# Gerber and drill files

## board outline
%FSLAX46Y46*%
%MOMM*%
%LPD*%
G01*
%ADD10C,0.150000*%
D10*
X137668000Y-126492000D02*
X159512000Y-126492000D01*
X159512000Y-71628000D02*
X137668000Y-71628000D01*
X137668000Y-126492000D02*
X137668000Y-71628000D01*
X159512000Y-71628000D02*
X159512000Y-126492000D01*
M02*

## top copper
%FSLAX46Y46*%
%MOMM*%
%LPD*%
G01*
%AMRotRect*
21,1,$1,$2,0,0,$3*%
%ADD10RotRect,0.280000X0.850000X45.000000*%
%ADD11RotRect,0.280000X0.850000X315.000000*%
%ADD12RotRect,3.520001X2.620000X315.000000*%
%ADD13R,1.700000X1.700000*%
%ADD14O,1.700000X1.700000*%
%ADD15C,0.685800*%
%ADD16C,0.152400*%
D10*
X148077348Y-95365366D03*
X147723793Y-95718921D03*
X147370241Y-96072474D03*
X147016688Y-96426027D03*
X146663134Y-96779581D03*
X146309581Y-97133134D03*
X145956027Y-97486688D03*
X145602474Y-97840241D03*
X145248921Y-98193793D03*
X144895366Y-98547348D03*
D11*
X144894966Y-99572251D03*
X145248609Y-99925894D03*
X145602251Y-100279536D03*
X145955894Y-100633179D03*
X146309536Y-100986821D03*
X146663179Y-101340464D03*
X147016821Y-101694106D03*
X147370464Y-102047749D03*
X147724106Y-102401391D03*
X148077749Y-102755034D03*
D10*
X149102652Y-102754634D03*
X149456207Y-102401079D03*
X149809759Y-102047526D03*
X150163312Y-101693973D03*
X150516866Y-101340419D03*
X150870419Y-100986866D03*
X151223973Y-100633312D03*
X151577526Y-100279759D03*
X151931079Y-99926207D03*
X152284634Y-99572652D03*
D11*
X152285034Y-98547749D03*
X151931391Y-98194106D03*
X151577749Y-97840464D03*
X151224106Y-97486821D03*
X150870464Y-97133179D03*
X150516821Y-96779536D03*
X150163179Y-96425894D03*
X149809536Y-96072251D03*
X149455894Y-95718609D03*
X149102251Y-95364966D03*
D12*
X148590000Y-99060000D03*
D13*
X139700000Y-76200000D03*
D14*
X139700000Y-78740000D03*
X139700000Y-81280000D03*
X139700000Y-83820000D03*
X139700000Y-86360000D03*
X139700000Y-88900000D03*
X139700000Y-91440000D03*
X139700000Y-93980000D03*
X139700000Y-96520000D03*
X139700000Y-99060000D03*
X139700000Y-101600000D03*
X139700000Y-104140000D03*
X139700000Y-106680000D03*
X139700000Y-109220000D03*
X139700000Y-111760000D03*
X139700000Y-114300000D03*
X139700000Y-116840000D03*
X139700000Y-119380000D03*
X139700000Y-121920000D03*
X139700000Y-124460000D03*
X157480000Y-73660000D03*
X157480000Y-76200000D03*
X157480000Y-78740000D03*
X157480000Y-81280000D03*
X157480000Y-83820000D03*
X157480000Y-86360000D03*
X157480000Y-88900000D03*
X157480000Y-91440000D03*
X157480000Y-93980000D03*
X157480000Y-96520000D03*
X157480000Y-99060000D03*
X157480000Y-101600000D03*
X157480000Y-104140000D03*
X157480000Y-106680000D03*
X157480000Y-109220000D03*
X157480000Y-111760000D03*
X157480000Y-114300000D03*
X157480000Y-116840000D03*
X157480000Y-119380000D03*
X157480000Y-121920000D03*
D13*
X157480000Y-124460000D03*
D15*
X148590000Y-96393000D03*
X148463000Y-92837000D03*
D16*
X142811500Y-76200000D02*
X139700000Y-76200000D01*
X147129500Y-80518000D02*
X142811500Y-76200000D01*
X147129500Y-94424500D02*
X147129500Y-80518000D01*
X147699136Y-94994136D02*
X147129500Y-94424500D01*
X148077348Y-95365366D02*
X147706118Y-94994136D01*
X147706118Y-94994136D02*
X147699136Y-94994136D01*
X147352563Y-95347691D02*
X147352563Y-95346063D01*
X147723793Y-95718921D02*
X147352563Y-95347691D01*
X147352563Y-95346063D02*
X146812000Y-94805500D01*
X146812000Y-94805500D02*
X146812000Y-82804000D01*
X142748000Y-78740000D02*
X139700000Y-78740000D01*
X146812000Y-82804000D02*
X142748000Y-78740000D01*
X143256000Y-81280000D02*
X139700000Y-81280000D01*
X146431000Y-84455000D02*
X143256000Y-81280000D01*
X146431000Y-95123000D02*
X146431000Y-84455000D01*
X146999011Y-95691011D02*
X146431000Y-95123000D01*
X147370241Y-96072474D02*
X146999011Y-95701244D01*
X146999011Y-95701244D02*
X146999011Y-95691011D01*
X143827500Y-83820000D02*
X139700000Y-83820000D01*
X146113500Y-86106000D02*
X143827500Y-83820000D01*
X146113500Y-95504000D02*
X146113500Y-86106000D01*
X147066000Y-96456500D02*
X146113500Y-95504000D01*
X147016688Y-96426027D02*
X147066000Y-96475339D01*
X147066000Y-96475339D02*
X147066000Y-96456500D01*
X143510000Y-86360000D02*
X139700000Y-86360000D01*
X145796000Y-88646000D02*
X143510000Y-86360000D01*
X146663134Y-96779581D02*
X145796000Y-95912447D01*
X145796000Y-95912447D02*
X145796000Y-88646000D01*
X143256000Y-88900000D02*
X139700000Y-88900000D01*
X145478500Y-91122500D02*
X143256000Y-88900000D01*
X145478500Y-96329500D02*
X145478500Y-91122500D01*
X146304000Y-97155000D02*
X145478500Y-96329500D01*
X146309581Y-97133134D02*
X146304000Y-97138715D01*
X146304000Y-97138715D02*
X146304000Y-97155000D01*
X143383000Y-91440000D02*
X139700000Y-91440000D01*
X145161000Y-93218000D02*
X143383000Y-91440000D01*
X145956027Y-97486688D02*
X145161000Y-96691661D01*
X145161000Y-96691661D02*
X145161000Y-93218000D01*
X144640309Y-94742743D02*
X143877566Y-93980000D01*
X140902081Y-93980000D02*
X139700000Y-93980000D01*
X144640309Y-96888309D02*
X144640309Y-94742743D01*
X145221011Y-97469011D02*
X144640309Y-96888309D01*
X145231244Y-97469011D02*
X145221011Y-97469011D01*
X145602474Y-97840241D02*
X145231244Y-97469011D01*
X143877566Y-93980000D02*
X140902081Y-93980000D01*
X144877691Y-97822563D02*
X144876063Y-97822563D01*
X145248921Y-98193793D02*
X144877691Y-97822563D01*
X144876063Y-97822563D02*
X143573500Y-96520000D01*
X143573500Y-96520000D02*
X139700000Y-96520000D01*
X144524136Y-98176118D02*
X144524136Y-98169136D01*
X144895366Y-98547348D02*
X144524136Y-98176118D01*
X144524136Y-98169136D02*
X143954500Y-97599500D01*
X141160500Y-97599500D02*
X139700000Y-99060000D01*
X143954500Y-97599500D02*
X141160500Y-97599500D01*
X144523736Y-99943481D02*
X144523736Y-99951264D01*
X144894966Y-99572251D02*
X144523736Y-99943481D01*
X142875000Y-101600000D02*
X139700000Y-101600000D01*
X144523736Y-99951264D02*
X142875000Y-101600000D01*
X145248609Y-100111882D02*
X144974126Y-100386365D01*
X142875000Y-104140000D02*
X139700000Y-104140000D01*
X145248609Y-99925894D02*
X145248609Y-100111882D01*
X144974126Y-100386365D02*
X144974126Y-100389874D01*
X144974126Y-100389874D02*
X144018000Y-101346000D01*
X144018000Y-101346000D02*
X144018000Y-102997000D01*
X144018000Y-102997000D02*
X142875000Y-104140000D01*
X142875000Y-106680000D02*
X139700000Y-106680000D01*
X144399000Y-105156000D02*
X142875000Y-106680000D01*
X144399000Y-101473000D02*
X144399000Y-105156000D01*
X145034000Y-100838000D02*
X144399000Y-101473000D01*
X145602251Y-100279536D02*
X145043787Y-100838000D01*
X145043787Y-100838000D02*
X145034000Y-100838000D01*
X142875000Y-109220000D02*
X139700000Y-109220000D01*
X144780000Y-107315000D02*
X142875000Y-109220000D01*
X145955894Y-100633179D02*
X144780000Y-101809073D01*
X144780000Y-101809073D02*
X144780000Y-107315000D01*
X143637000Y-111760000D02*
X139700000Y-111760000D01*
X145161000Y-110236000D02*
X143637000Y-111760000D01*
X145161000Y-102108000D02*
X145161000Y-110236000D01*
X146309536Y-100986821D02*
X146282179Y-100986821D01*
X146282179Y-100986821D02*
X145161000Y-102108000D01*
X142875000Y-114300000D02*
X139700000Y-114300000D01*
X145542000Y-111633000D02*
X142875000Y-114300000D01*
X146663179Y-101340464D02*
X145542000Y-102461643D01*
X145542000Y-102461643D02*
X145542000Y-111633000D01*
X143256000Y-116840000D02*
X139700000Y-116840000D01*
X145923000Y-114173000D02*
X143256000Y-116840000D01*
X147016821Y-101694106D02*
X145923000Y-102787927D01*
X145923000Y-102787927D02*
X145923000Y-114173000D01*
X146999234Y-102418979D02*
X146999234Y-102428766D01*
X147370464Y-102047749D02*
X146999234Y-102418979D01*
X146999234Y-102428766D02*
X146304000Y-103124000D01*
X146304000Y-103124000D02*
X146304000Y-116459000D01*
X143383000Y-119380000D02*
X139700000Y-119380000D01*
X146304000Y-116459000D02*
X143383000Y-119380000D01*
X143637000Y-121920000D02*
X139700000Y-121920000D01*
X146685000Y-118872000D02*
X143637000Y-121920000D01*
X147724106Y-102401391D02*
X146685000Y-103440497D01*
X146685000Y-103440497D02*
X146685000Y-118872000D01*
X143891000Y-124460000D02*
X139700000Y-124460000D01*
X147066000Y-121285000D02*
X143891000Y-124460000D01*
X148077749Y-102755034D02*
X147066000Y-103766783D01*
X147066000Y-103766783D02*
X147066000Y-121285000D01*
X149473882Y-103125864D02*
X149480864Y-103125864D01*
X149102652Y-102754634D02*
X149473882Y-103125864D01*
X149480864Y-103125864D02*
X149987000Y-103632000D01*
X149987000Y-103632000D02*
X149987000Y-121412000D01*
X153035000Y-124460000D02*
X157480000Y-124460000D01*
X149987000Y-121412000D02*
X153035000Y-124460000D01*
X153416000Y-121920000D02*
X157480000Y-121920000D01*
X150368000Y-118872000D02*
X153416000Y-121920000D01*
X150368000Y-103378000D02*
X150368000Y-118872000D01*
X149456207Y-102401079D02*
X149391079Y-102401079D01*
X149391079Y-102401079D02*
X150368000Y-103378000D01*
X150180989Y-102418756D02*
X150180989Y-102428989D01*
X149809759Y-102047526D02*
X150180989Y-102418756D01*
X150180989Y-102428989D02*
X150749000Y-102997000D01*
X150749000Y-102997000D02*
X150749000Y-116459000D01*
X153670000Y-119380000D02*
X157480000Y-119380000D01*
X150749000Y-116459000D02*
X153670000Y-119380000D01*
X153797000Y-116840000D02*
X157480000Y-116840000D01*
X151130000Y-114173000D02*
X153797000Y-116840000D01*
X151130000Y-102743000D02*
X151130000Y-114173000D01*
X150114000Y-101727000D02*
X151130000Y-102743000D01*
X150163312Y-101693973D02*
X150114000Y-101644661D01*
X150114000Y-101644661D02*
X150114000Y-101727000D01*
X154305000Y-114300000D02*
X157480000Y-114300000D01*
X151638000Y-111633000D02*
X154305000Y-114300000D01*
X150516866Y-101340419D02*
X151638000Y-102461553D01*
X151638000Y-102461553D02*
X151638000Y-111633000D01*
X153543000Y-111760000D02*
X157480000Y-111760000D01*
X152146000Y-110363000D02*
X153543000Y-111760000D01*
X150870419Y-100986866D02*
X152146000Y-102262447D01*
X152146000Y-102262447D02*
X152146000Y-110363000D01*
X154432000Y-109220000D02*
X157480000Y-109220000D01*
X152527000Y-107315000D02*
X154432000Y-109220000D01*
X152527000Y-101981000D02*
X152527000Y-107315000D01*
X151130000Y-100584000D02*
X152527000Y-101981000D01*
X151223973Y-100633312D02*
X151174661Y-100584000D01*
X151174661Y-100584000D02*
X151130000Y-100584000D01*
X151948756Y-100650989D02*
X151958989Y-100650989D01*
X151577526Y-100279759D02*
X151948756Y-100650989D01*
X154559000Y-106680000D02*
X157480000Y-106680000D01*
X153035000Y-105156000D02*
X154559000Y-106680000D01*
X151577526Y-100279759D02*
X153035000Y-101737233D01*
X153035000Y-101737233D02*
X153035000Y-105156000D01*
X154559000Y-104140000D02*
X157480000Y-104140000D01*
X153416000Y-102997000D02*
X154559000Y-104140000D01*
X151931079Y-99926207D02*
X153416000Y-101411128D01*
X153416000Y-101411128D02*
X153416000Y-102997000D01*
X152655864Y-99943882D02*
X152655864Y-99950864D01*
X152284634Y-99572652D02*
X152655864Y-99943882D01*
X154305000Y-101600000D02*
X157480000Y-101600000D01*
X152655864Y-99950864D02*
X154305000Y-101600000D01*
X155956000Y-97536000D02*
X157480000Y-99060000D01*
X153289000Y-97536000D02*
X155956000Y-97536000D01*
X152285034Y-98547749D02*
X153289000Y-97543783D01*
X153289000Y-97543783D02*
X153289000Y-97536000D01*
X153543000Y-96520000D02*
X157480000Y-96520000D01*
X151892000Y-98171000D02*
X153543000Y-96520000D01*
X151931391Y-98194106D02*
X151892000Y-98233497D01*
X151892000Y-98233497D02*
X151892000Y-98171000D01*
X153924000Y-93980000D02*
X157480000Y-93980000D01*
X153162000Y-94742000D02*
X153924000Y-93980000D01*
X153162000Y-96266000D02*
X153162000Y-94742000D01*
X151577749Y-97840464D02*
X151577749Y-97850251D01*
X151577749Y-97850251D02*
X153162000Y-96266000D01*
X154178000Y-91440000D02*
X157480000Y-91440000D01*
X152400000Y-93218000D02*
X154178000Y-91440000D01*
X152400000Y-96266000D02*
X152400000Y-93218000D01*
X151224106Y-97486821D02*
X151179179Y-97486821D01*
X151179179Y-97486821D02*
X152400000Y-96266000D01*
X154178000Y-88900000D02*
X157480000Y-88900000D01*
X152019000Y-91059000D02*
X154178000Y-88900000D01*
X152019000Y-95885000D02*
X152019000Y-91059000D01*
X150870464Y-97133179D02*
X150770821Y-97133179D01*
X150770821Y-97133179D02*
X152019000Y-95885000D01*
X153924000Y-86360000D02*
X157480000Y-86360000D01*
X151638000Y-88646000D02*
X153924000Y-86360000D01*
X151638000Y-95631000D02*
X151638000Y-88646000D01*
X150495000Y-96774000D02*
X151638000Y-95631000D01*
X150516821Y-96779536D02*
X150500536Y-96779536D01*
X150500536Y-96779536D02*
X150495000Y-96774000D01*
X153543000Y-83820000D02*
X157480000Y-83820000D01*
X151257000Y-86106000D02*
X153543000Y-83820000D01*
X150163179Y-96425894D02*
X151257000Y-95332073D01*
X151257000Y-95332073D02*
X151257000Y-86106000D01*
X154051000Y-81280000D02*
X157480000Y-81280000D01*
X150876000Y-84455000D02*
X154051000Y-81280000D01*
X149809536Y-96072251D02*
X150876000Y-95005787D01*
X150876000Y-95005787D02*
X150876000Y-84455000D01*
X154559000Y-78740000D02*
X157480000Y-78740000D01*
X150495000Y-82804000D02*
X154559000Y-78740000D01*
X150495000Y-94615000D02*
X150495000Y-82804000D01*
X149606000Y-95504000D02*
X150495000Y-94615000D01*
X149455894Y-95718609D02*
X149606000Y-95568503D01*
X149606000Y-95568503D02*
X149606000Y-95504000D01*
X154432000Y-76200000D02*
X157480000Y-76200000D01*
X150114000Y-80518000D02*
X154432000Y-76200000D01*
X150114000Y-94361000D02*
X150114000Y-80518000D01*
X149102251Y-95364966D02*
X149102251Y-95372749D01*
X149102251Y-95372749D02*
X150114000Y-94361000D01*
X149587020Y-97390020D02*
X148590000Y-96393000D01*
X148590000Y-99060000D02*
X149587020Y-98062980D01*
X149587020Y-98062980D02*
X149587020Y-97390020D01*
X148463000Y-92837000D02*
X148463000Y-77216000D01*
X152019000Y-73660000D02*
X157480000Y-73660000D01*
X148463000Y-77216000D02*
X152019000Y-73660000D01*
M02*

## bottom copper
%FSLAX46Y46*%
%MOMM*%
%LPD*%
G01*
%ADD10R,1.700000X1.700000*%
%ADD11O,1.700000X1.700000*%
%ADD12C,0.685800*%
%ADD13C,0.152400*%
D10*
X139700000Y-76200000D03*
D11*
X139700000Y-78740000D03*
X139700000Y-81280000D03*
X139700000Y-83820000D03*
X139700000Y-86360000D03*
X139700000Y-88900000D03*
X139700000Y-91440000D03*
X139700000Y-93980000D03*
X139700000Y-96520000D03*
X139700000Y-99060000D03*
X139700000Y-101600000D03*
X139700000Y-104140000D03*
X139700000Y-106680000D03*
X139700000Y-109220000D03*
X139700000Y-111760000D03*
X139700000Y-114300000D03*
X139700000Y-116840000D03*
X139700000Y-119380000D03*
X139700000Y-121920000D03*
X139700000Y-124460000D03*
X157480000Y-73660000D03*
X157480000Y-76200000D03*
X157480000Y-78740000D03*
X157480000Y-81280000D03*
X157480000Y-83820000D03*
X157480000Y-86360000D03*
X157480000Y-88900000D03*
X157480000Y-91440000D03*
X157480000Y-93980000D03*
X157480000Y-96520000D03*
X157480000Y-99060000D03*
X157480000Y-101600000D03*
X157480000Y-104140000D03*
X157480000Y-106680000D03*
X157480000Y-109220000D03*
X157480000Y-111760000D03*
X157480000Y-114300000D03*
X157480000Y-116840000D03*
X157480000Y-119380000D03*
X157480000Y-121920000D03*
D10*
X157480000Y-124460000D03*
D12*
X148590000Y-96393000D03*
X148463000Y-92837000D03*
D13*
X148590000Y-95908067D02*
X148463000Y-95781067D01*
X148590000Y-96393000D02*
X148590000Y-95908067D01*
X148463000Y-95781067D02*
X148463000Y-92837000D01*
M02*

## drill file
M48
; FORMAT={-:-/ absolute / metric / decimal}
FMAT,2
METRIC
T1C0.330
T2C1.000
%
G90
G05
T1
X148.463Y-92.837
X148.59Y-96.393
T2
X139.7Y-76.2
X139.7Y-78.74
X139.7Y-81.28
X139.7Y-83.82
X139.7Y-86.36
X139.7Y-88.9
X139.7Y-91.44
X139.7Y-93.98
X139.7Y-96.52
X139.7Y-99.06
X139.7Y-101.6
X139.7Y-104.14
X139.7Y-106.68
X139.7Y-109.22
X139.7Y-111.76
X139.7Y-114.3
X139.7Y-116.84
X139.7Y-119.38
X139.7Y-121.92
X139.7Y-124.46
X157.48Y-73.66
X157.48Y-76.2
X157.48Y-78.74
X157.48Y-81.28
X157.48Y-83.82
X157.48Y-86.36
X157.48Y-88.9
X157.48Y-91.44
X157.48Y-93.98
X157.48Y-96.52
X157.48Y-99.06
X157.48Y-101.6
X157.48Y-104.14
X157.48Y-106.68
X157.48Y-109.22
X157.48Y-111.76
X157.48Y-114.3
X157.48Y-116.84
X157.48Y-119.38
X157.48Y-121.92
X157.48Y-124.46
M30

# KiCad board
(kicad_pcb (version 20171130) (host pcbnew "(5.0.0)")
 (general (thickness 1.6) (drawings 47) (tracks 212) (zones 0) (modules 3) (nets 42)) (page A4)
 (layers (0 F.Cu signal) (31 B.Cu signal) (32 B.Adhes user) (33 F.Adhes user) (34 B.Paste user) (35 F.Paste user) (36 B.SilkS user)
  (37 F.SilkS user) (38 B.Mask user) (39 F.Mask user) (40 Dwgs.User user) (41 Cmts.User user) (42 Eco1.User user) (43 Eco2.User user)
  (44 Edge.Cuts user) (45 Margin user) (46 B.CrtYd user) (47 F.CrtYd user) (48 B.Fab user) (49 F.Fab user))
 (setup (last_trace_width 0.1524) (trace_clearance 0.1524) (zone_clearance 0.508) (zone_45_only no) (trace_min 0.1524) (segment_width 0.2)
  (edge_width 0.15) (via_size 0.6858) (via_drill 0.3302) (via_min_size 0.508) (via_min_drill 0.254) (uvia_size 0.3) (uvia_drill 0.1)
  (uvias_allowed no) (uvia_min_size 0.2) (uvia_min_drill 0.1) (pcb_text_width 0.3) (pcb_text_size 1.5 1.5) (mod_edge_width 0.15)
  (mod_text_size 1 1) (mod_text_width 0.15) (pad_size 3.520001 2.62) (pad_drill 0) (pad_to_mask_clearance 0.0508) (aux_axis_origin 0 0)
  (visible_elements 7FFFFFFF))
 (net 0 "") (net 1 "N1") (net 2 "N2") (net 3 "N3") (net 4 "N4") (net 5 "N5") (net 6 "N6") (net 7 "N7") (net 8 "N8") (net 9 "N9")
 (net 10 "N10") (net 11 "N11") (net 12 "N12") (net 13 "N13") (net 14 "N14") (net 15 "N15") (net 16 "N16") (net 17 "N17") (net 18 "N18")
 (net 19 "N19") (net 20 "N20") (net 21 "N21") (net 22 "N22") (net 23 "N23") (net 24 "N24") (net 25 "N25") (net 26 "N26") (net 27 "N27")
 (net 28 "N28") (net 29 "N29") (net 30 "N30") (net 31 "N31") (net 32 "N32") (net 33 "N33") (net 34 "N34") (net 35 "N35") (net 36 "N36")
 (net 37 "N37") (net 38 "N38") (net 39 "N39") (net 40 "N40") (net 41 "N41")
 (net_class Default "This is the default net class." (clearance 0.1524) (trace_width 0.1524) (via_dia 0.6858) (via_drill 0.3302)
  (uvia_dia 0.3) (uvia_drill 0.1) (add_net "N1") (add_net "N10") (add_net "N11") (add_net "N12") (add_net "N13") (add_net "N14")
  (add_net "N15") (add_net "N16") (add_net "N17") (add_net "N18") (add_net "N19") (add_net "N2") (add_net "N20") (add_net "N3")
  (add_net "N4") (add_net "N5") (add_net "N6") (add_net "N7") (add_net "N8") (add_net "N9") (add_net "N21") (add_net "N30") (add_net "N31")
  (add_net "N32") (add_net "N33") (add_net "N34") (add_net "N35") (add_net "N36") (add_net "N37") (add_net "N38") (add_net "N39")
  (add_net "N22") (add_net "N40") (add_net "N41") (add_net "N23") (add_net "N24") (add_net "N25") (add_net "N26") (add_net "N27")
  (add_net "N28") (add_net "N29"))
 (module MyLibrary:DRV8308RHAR (layer F.Cu) (at 148.59 99.06 315)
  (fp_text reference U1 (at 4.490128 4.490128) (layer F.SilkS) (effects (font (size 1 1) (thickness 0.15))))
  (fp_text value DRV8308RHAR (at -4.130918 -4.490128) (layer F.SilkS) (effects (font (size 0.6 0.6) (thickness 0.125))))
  (pad 1 smd rect (at -2.975 -2.250001 45) (size 0.28 0.85) (layers F.Cu F.Paste F.Mask) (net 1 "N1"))
  (pad 2 smd rect (at -2.975 -1.749999 45) (size 0.28 0.85) (layers F.Cu F.Paste F.Mask) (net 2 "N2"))
  (pad 3 smd rect (at -2.975 -1.25 45) (size 0.28 0.85) (layers F.Cu F.Paste F.Mask) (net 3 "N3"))
  (pad 4 smd rect (at -2.975 -0.750001 45) (size 0.28 0.85) (layers F.Cu F.Paste F.Mask) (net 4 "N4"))
  (pad 5 smd rect (at -2.975 -0.25 45) (size 0.28 0.85) (layers F.Cu F.Paste F.Mask) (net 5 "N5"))
  (pad 6 smd rect (at -2.975 0.25 45) (size 0.28 0.85) (layers F.Cu F.Paste F.Mask) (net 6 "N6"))
  (pad 7 smd rect (at -2.975 0.750001 45) (size 0.28 0.85) (layers F.Cu F.Paste F.Mask) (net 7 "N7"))
  (pad 8 smd rect (at -2.975 1.25 45) (size 0.28 0.85) (layers F.Cu F.Paste F.Mask) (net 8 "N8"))
  (pad 9 smd rect (at -2.975 1.749999 45) (size 0.28 0.85) (layers F.Cu F.Paste F.Mask) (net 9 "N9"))
  (pad 10 smd rect (at -2.975 2.250001 45) (size 0.28 0.85) (layers F.Cu F.Paste F.Mask) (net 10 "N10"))
  (pad 11 smd rect (at -2.250567 2.975 315) (size 0.28 0.85) (layers F.Cu F.Paste F.Mask) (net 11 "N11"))
  (pad 12 smd rect (at -1.750441 2.975 315) (size 0.28 0.85) (layers F.Cu F.Paste F.Mask) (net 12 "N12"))
  (pad 13 smd rect (at -1.250315 2.975 315) (size 0.28 0.85) (layers F.Cu F.Paste F.Mask) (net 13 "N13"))
  (pad 14 smd rect (at -0.750189 2.975 315) (size 0.28 0.85) (layers F.Cu F.Paste F.Mask) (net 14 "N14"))
  (pad 15 smd rect (at -0.250063 2.975 315) (size 0.28 0.85) (layers F.Cu F.Paste F.Mask) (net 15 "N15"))
  (pad 16 smd rect (at 0.250063 2.975 315) (size 0.28 0.85) (layers F.Cu F.Paste F.Mask) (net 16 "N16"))
  (pad 17 smd rect (at 0.750189 2.975 315) (size 0.28 0.85) (layers F.Cu F.Paste F.Mask) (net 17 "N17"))
  (pad 18 smd rect (at 1.250315 2.975 315) (size 0.28 0.85) (layers F.Cu F.Paste F.Mask) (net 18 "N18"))
  (pad 19 smd rect (at 1.750441 2.975 315) (size 0.28 0.85) (layers F.Cu F.Paste F.Mask) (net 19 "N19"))
  (pad 20 smd rect (at 2.250567 2.975 315) (size 0.28 0.85) (layers F.Cu F.Paste F.Mask) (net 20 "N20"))
  (pad 21 smd rect (at 2.975 2.250001 45) (size 0.28 0.85) (layers F.Cu F.Paste F.Mask) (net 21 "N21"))
  (pad 22 smd rect (at 2.975 1.749999 45) (size 0.28 0.85) (layers F.Cu F.Paste F.Mask) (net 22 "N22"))
  (pad 23 smd rect (at 2.975 1.25 45) (size 0.28 0.85) (layers F.Cu F.Paste F.Mask) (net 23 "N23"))
  (pad 24 smd rect (at 2.975 0.750001 45) (size 0.28 0.85) (layers F.Cu F.Paste F.Mask) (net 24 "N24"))
  (pad 25 smd rect (at 2.975 0.25 45) (size 0.28 0.85) (layers F.Cu F.Paste F.Mask) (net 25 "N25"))
  (pad 26 smd rect (at 2.975 -0.25 45) (size 0.28 0.85) (layers F.Cu F.Paste F.Mask) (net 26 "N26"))
  (pad 27 smd rect (at 2.975 -0.750001 45) (size 0.28 0.85) (layers F.Cu F.Paste F.Mask) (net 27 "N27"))
  (pad 28 smd rect (at 2.975 -1.25 45) (size 0.28 0.85) (layers F.Cu F.Paste F.Mask) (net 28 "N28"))
  (pad 29 smd rect (at 2.975 -1.749999 45) (size 0.28 0.85) (layers F.Cu F.Paste F.Mask) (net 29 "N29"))
  (pad 30 smd rect (at 2.975 -2.250001 45) (size 0.28 0.85) (layers F.Cu F.Paste F.Mask) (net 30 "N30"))
  (pad 31 smd rect (at 2.250567 -2.975 315) (size 0.28 0.85) (layers F.Cu F.Paste F.Mask) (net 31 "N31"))
  (pad 32 smd rect (at 1.750441 -2.975 315) (size 0.28 0.85) (layers F.Cu F.Paste F.Mask) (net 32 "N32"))
  (pad 33 smd rect (at 1.250315 -2.975 315) (size 0.28 0.85) (layers F.Cu F.Paste F.Mask) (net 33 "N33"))
  (pad 34 smd rect (at 0.750189 -2.975 315) (size 0.28 0.85) (layers F.Cu F.Paste F.Mask) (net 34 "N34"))
  (pad 35 smd rect (at 0.250063 -2.975 315) (size 0.28 0.85) (layers F.Cu F.Paste F.Mask) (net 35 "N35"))
  (pad 36 smd rect (at -0.250063 -2.975 315) (size 0.28 0.85) (layers F.Cu F.Paste F.Mask) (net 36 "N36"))
  (pad 37 smd rect (at -0.750189 -2.975 315) (size 0.28 0.85) (layers F.Cu F.Paste F.Mask) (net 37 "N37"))
  (pad 38 smd rect (at -1.250315 -2.975 315) (size 0.28 0.85) (layers F.Cu F.Paste F.Mask) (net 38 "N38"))
  (pad 39 smd rect (at -1.750441 -2.975 315) (size 0.28 0.85) (layers F.Cu F.Paste F.Mask) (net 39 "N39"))
  (pad 40 smd rect (at -2.250567 -2.975 315) (size 0.28 0.85) (layers F.Cu F.Paste F.Mask) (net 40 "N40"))
  (pad 41 smd rect (at 0 0 315) (size 3.520001 2.62) (layers F.Cu F.Paste F.Mask) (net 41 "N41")))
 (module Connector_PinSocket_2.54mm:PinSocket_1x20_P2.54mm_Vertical (layer F.Cu) (at 139.7 76.2)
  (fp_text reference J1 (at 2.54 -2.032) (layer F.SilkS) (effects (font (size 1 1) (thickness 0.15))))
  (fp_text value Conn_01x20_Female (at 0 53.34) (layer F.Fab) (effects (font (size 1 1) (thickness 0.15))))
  (pad 1 thru_hole rect (at 0 0) (size 1.7 1.7) (drill 1) (layers *.Cu *.Mask) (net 1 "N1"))
  (pad 2 thru_hole oval (at 0 2.54) (size 1.7 1.7) (drill 1) (layers *.Cu *.Mask) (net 2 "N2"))
  (pad 3 thru_hole oval (at 0 5.08) (size 1.7 1.7) (drill 1) (layers *.Cu *.Mask) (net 3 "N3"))
  (pad 4 thru_hole oval (at 0 7.62) (size 1.7 1.7) (drill 1) (layers *.Cu *.Mask) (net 4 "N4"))
  (pad 5 thru_hole oval (at 0 10.16) (size 1.7 1.7) (drill 1) (layers *.Cu *.Mask) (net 5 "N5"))
  (pad 6 thru_hole oval (at 0 12.7) (size 1.7 1.7) (drill 1) (layers *.Cu *.Mask) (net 6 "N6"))
  (pad 7 thru_hole oval (at 0 15.24) (size 1.7 1.7) (drill 1) (layers *.Cu *.Mask) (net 7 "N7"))
  (pad 8 thru_hole oval (at 0 17.78) (size 1.7 1.7) (drill 1) (layers *.Cu *.Mask) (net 8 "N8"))
  (pad 9 thru_hole oval (at 0 20.32) (size 1.7 1.7) (drill 1) (layers *.Cu *.Mask) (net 9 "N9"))
  (pad 10 thru_hole oval (at 0 22.86) (size 1.7 1.7) (drill 1) (layers *.Cu *.Mask) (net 10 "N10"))
  (pad 11 thru_hole oval (at 0 25.4) (size 1.7 1.7) (drill 1) (layers *.Cu *.Mask) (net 11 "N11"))
  (pad 12 thru_hole oval (at 0 27.94) (size 1.7 1.7) (drill 1) (layers *.Cu *.Mask) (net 12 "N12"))
  (pad 13 thru_hole oval (at 0 30.48) (size 1.7 1.7) (drill 1) (layers *.Cu *.Mask) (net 13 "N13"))
  (pad 14 thru_hole oval (at 0 33.02) (size 1.7 1.7) (drill 1) (layers *.Cu *.Mask) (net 14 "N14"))
  (pad 15 thru_hole oval (at 0 35.56) (size 1.7 1.7) (drill 1) (layers *.Cu *.Mask) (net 15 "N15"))
  (pad 16 thru_hole oval (at 0 38.1) (size 1.7 1.7) (drill 1) (layers *.Cu *.Mask) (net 16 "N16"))
  (pad 17 thru_hole oval (at 0 40.64) (size 1.7 1.7) (drill 1) (layers *.Cu *.Mask) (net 17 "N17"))
  (pad 18 thru_hole oval (at 0 43.18) (size 1.7 1.7) (drill 1) (layers *.Cu *.Mask) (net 18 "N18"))
  (pad 19 thru_hole oval (at 0 45.72) (size 1.7 1.7) (drill 1) (layers *.Cu *.Mask) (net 19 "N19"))
  (pad 20 thru_hole oval (at 0 48.26) (size 1.7 1.7) (drill 1) (layers *.Cu *.Mask) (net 20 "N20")))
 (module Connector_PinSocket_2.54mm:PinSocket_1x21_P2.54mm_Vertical (layer F.Cu) (at 157.48 124.46 180)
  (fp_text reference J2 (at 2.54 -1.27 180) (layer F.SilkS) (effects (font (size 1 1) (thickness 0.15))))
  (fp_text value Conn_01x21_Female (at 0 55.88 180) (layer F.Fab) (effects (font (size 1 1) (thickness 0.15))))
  (pad 21 thru_hole oval (at 0 50.8 180) (size 1.7 1.7) (drill 1) (layers *.Cu *.Mask) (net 41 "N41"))
  (pad 20 thru_hole oval (at 0 48.26 180) (size 1.7 1.7) (drill 1) (layers *.Cu *.Mask) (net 40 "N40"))
  (pad 19 thru_hole oval (at 0 45.72 180) (size 1.7 1.7) (drill 1) (layers *.Cu *.Mask) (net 39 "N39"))
  (pad 18 thru_hole oval (at 0 43.18 180) (size 1.7 1.7) (drill 1) (layers *.Cu *.Mask) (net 38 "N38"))
  (pad 17 thru_hole oval (at 0 40.64 180) (size 1.7 1.7) (drill 1) (layers *.Cu *.Mask) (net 37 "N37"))
  (pad 16 thru_hole oval (at 0 38.1 180) (size 1.7 1.7) (drill 1) (layers *.Cu *.Mask) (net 36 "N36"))
  (pad 15 thru_hole oval (at 0 35.56 180) (size 1.7 1.7) (drill 1) (layers *.Cu *.Mask) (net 35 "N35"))
  (pad 14 thru_hole oval (at 0 33.02 180) (size 1.7 1.7) (drill 1) (layers *.Cu *.Mask) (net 34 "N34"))
  (pad 13 thru_hole oval (at 0 30.48 180) (size 1.7 1.7) (drill 1) (layers *.Cu *.Mask) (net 33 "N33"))
  (pad 12 thru_hole oval (at 0 27.94 180) (size 1.7 1.7) (drill 1) (layers *.Cu *.Mask) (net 32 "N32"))
  (pad 11 thru_hole oval (at 0 25.4 180) (size 1.7 1.7) (drill 1) (layers *.Cu *.Mask) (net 31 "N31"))
  (pad 10 thru_hole oval (at 0 22.86 180) (size 1.7 1.7) (drill 1) (layers *.Cu *.Mask) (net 30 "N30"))
  (pad 9 thru_hole oval (at 0 20.32 180) (size 1.7 1.7) (drill 1) (layers *.Cu *.Mask) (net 29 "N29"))
  (pad 8 thru_hole oval (at 0 17.78 180) (size 1.7 1.7) (drill 1) (layers *.Cu *.Mask) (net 28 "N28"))
  (pad 7 thru_hole oval (at 0 15.24 180) (size 1.7 1.7) (drill 1) (layers *.Cu *.Mask) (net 27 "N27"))
  (pad 6 thru_hole oval (at 0 12.7 180) (size 1.7 1.7) (drill 1) (layers *.Cu *.Mask) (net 26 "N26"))
  (pad 5 thru_hole oval (at 0 10.16 180) (size 1.7 1.7) (drill 1) (layers *.Cu *.Mask) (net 25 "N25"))
  (pad 4 thru_hole oval (at 0 7.62 180) (size 1.7 1.7) (drill 1) (layers *.Cu *.Mask) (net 24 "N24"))
  (pad 3 thru_hole oval (at 0 5.08 180) (size 1.7 1.7) (drill 1) (layers *.Cu *.Mask) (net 23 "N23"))
  (pad 2 thru_hole oval (at 0 2.54 180) (size 1.7 1.7) (drill 1) (layers *.Cu *.Mask) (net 22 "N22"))
  (pad 1 thru_hole rect (at 0 0 180) (size 1.7 1.7) (drill 1) (layers *.Cu *.Mask) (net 21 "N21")))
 (gr_line (start 137.668 126.492) (end 159.512 126.492) (layer Edge.Cuts) (width 0.15))
 (gr_line (start 159.512 71.628) (end 137.668 71.628) (layer Edge.Cuts) (width 0.15))
 (gr_line (start 137.668 126.492) (end 137.668 71.628) (layer Edge.Cuts) (width 0.15))
 (gr_line (start 159.512 71.628) (end 159.512 126.492) (layer Edge.Cuts) (width 0.15))
 (segment (start 142.8115 76.2) (end 139.7 76.2) (width 0.1524) (layer F.Cu) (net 1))
 (segment (start 147.1295 80.518) (end 142.8115 76.2) (width 0.1524) (layer F.Cu) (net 1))
 (segment (start 147.1295 94.4245) (end 147.1295 80.518) (width 0.1524) (layer F.Cu) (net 1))
 (segment (start 147.699136 94.994136) (end 147.1295 94.4245) (width 0.1524) (layer F.Cu) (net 1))
 (segment (start 148.077348 95.365366) (end 147.706118 94.994136) (width 0.1524) (layer F.Cu) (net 1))
 (segment (start 147.706118 94.994136) (end 147.699136 94.994136) (width 0.1524) (layer F.Cu) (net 1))
 (segment (start 147.352563 95.347691) (end 147.352563 95.346063) (width 0.1524) (layer F.Cu) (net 2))
 (segment (start 147.723793 95.718921) (end 147.352563 95.347691) (width 0.1524) (layer F.Cu) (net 2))
 (segment (start 147.352563 95.346063) (end 146.812 94.8055) (width 0.1524) (layer F.Cu) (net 2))
 (segment (start 146.812 94.8055) (end 146.812 82.804) (width 0.1524) (layer F.Cu) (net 2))
 (segment (start 142.748 78.74) (end 139.7 78.74) (width 0.1524) (layer F.Cu) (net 2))
 (segment (start 146.812 82.804) (end 142.748 78.74) (width 0.1524) (layer F.Cu) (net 2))
 (segment (start 143.256 81.28) (end 139.7 81.28) (width 0.1524) (layer F.Cu) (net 3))
 (segment (start 146.431 84.455) (end 143.256 81.28) (width 0.1524) (layer F.Cu) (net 3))
 (segment (start 146.431 95.123) (end 146.431 84.455) (width 0.1524) (layer F.Cu) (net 3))
 (segment (start 146.999011 95.691011) (end 146.431 95.123) (width 0.1524) (layer F.Cu) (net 3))
 (segment (start 147.370241 96.072474) (end 146.999011 95.701244) (width 0.1524) (layer F.Cu) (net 3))
 (segment (start 146.999011 95.701244) (end 146.999011 95.691011) (width 0.1524) (layer F.Cu) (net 3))
 (segment (start 143.8275 83.82) (end 139.7 83.82) (width 0.1524) (layer F.Cu) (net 4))
 (segment (start 146.1135 86.106) (end 143.8275 83.82) (width 0.1524) (layer F.Cu) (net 4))
 (segment (start 146.1135 95.504) (end 146.1135 86.106) (width 0.1524) (layer F.Cu) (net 4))
 (segment (start 147.066 96.4565) (end 146.1135 95.504) (width 0.1524) (layer F.Cu) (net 4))
 (segment (start 147.016688 96.426027) (end 147.066 96.475339) (width 0.1524) (layer F.Cu) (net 4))
 (segment (start 147.066 96.475339) (end 147.066 96.4565) (width 0.1524) (layer F.Cu) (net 4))
 (segment (start 143.51 86.36) (end 139.7 86.36) (width 0.1524) (layer F.Cu) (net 5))
 (segment (start 145.796 88.646) (end 143.51 86.36) (width 0.1524) (layer F.Cu) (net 5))
 (segment (start 146.663134 96.779581) (end 145.796 95.912447) (width 0.1524) (layer F.Cu) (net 5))
 (segment (start 145.796 95.912447) (end 145.796 88.646) (width 0.1524) (layer F.Cu) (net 5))
 (segment (start 143.256 88.9) (end 139.7 88.9) (width 0.1524) (layer F.Cu) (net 6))
 (segment (start 145.4785 91.1225) (end 143.256 88.9) (width 0.1524) (layer F.Cu) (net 6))
 (segment (start 145.4785 96.3295) (end 145.4785 91.1225) (width 0.1524) (layer F.Cu) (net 6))
 (segment (start 146.304 97.155) (end 145.4785 96.3295) (width 0.1524) (layer F.Cu) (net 6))
 (segment (start 146.309581 97.133134) (end 146.304 97.138715) (width 0.1524) (layer F.Cu) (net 6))
 (segment (start 146.304 97.138715) (end 146.304 97.155) (width 0.1524) (layer F.Cu) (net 6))
 (segment (start 143.383 91.44) (end 139.7 91.44) (width 0.1524) (layer F.Cu) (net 7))
 (segment (start 145.161 93.218) (end 143.383 91.44) (width 0.1524) (layer F.Cu) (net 7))
 (segment (start 145.956027 97.486688) (end 145.161 96.691661) (width 0.1524) (layer F.Cu) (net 7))
 (segment (start 145.161 96.691661) (end 145.161 93.218) (width 0.1524) (layer F.Cu) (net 7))
 (segment (start 144.640309 94.742743) (end 143.877566 93.98) (width 0.1524) (layer F.Cu) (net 8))
 (segment (start 140.902081 93.98) (end 139.7 93.98) (width 0.1524) (layer F.Cu) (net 8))
 (segment (start 144.640309 96.888309) (end 144.640309 94.742743) (width 0.1524) (layer F.Cu) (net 8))
 (segment (start 145.221011 97.469011) (end 144.640309 96.888309) (width 0.1524) (layer F.Cu) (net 8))
 (segment (start 145.231244 97.469011) (end 145.221011 97.469011) (width 0.1524) (layer F.Cu) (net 8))
 (segment (start 145.602474 97.840241) (end 145.231244 97.469011) (width 0.1524) (layer F.Cu) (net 8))
 (segment (start 143.877566 93.98) (end 140.902081 93.98) (width 0.1524) (layer F.Cu) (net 8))
 (segment (start 144.877691 97.822563) (end 144.876063 97.822563) (width 0.1524) (layer F.Cu) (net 9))
 (segment (start 145.248921 98.193793) (end 144.877691 97.822563) (width 0.1524) (layer F.Cu) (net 9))
 (segment (start 144.876063 97.822563) (end 143.5735 96.52) (width 0.1524) (layer F.Cu) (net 9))
 (segment (start 143.5735 96.52) (end 139.7 96.52) (width 0.1524) (layer F.Cu) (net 9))
 (segment (start 144.524136 98.176118) (end 144.524136 98.169136) (width 0.1524) (layer F.Cu) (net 10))
 (segment (start 144.895366 98.547348) (end 144.524136 98.176118) (width 0.1524) (layer F.Cu) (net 10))
 (segment (start 144.524136 98.169136) (end 143.9545 97.5995) (width 0.1524) (layer F.Cu) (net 10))
 (segment (start 141.1605 97.5995) (end 139.7 99.06) (width 0.1524) (layer F.Cu) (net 10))
 (segment (start 143.9545 97.5995) (end 141.1605 97.5995) (width 0.1524) (layer F.Cu) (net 10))
 (segment (start 144.523736 99.943481) (end 144.523736 99.951264) (width 0.1524) (layer F.Cu) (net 11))
 (segment (start 144.894966 99.572251) (end 144.523736 99.943481) (width 0.1524) (layer F.Cu) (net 11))
 (segment (start 142.875 101.6) (end 139.7 101.6) (width 0.1524) (layer F.Cu) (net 11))
 (segment (start 144.523736 99.951264) (end 142.875 101.6) (width 0.1524) (layer F.Cu) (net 11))
 (segment (start 145.248609 100.111882) (end 144.974126 100.386365) (width 0.1524) (layer F.Cu) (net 12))
 (segment (start 142.875 104.14) (end 139.7 104.14) (width 0.1524) (layer F.Cu) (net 12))
 (segment (start 145.248609 99.925894) (end 145.248609 100.111882) (width 0.1524) (layer F.Cu) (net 12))
 (segment (start 144.974126 100.386365) (end 144.974126 100.389874) (width 0.1524) (layer F.Cu) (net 12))
 (segment (start 144.974126 100.389874) (end 144.018 101.346) (width 0.1524) (layer F.Cu) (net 12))
 (segment (start 144.018 101.346) (end 144.018 102.997) (width 0.1524) (layer F.Cu) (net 12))
 (segment (start 144.018 102.997) (end 142.875 104.14) (width 0.1524) (layer F.Cu) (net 12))
 (segment (start 142.875 106.68) (end 139.7 106.68) (width 0.1524) (layer F.Cu) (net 13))
 (segment (start 144.399 105.156) (end 142.875 106.68) (width 0.1524) (layer F.Cu) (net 13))
 (segment (start 144.399 101.473) (end 144.399 105.156) (width 0.1524) (layer F.Cu) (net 13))
 (segment (start 145.034 100.838) (end 144.399 101.473) (width 0.1524) (layer F.Cu) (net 13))
 (segment (start 145.602251 100.279536) (end 145.043787 100.838) (width 0.1524) (layer F.Cu) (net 13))
 (segment (start 145.043787 100.838) (end 145.034 100.838) (width 0.1524) (layer F.Cu) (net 13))
 (segment (start 142.875 109.22) (end 139.7 109.22) (width 0.1524) (layer F.Cu) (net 14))
 (segment (start 144.78 107.315) (end 142.875 109.22) (width 0.1524) (layer F.Cu) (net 14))
 (segment (start 145.955894 100.633179) (end 144.78 101.809073) (width 0.1524) (layer F.Cu) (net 14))
 (segment (start 144.78 101.809073) (end 144.78 107.315) (width 0.1524) (layer F.Cu) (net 14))
 (segment (start 143.637 111.76) (end 139.7 111.76) (width 0.1524) (layer F.Cu) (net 15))
 (segment (start 145.161 110.236) (end 143.637 111.76) (width 0.1524) (layer F.Cu) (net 15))
 (segment (start 145.161 102.108) (end 145.161 110.236) (width 0.1524) (layer F.Cu) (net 15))
 (segment (start 146.309536 100.986821) (end 146.282179 100.986821) (width 0.1524) (layer F.Cu) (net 15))
 (segment (start 146.282179 100.986821) (end 145.161 102.108) (width 0.1524) (layer F.Cu) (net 15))
 (segment (start 142.875 114.3) (end 139.7 114.3) (width 0.1524) (layer F.Cu) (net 16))
 (segment (start 145.542 111.633) (end 142.875 114.3) (width 0.1524) (layer F.Cu) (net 16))
 (segment (start 146.663179 101.340464) (end 145.542 102.461643) (width 0.1524) (layer F.Cu) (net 16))
 (segment (start 145.542 102.461643) (end 145.542 111.633) (width 0.1524) (layer F.Cu) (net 16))
 (segment (start 143.256 116.84) (end 139.7 116.84) (width 0.1524) (layer F.Cu) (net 17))
 (segment (start 145.923 114.173) (end 143.256 116.84) (width 0.1524) (layer F.Cu) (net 17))
 (segment (start 147.016821 101.694106) (end 145.923 102.787927) (width 0.1524) (layer F.Cu) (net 17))
 (segment (start 145.923 102.787927) (end 145.923 114.173) (width 0.1524) (layer F.Cu) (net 17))
 (segment (start 146.999234 102.418979) (end 146.999234 102.428766) (width 0.1524) (layer F.Cu) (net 18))
 (segment (start 147.370464 102.047749) (end 146.999234 102.418979) (width 0.1524) (layer F.Cu) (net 18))
 (segment (start 146.999234 102.428766) (end 146.304 103.124) (width 0.1524) (layer F.Cu) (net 18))
 (segment (start 146.304 103.124) (end 146.304 116.459) (width 0.1524) (layer F.Cu) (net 18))
 (segment (start 143.383 119.38) (end 139.7 119.38) (width 0.1524) (layer F.Cu) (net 18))
 (segment (start 146.304 116.459) (end 143.383 119.38) (width 0.1524) (layer F.Cu) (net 18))
 (segment (start 143.637 121.92) (end 139.7 121.92) (width 0.1524) (layer F.Cu) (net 19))
 (segment (start 146.685 118.872) (end 143.637 121.92) (width 0.1524) (layer F.Cu) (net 19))
 (segment (start 147.724106 102.401391) (end 146.685 103.440497) (width 0.1524) (layer F.Cu) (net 19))
 (segment (start 146.685 103.440497) (end 146.685 118.872) (width 0.1524) (layer F.Cu) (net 19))
 (segment (start 143.891 124.46) (end 139.7 124.46) (width 0.1524) (layer F.Cu) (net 20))
 (segment (start 147.066 121.285) (end 143.891 124.46) (width 0.1524) (layer F.Cu) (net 20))
 (segment (start 148.077749 102.755034) (end 147.066 103.766783) (width 0.1524) (layer F.Cu) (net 20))
 (segment (start 147.066 103.766783) (end 147.066 121.285) (width 0.1524) (layer F.Cu) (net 20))
 (segment (start 149.473882 103.125864) (end 149.480864 103.125864) (width 0.1524) (layer F.Cu) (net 21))
 (segment (start 149.102652 102.754634) (end 149.473882 103.125864) (width 0.1524) (layer F.Cu) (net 21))
 (segment (start 149.480864 103.125864) (end 149.987 103.632) (width 0.1524) (layer F.Cu) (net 21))
 (segment (start 149.987 103.632) (end 149.987 121.412) (width 0.1524) (layer F.Cu) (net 21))
 (segment (start 153.035 124.46) (end 157.48 124.46) (width 0.1524) (layer F.Cu) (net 21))
 (segment (start 149.987 121.412) (end 153.035 124.46) (width 0.1524) (layer F.Cu) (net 21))
 (segment (start 153.416 121.92) (end 157.48 121.92) (width 0.1524) (layer F.Cu) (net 22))
 (segment (start 150.368 118.872) (end 153.416 121.92) (width 0.1524) (layer F.Cu) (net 22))
 (segment (start 150.368 103.378) (end 150.368 118.872) (width 0.1524) (layer F.Cu) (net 22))
 (segment (start 149.456207 102.401079) (end 149.391079 102.401079) (width 0.1524) (layer F.Cu) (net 22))
 (segment (start 149.391079 102.401079) (end 150.368 103.378) (width 0.1524) (layer F.Cu) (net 22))
 (segment (start 150.180989 102.418756) (end 150.180989 102.428989) (width 0.1524) (layer F.Cu) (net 23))
 (segment (start 149.809759 102.047526) (end 150.180989 102.418756) (width 0.1524) (layer F.Cu) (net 23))
 (segment (start 150.180989 102.428989) (end 150.749 102.997) (width 0.1524) (layer F.Cu) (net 23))
 (segment (start 150.749 102.997) (end 150.749 116.459) (width 0.1524) (layer F.Cu) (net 23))
 (segment (start 153.67 119.38) (end 157.48 119.38) (width 0.1524) (layer F.Cu) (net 23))
 (segment (start 150.749 116.459) (end 153.67 119.38) (width 0.1524) (layer F.Cu) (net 23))
 (segment (start 153.797 116.84) (end 157.48 116.84) (width 0.1524) (layer F.Cu) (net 24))
 (segment (start 151.13 114.173) (end 153.797 116.84) (width 0.1524) (layer F.Cu) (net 24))
 (segment (start 151.13 102.743) (end 151.13 114.173) (width 0.1524) (layer F.Cu) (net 24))
 (segment (start 150.114 101.727) (end 151.13 102.743) (width 0.1524) (layer F.Cu) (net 24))
 (segment (start 150.163312 101.693973) (end 150.114 101.644661) (width 0.1524) (layer F.Cu) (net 24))
 (segment (start 150.114 101.644661) (end 150.114 101.727) (width 0.1524) (layer F.Cu) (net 24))
 (segment (start 154.305 114.3) (end 157.48 114.3) (width 0.1524) (layer F.Cu) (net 25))
 (segment (start 151.638 111.633) (end 154.305 114.3) (width 0.1524) (layer F.Cu) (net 25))
 (segment (start 150.516866 101.340419) (end 151.638 102.461553) (width 0.1524) (layer F.Cu) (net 25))
 (segment (start 151.638 102.461553) (end 151.638 111.633) (width 0.1524) (layer F.Cu) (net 25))
 (segment (start 153.543 111.76) (end 157.48 111.76) (width 0.1524) (layer F.Cu) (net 26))
 (segment (start 152.146 110.363) (end 153.543 111.76) (width 0.1524) (layer F.Cu) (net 26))
 (segment (start 150.870419 100.986866) (end 152.146 102.262447) (width 0.1524) (layer F.Cu) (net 26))
 (segment (start 152.146 102.262447) (end 152.146 110.363) (width 0.1524) (layer F.Cu) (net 26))
 (segment (start 154.432 109.22) (end 157.48 109.22) (width 0.1524) (layer F.Cu) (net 27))
 (segment (start 152.527 107.315) (end 154.432 109.22) (width 0.1524) (layer F.Cu) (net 27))
 (segment (start 152.527 101.981) (end 152.527 107.315) (width 0.1524) (layer F.Cu) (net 27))
 (segment (start 151.13 100.584) (end 152.527 101.981) (width 0.1524) (layer F.Cu) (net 27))
 (segment (start 151.223973 100.633312) (end 151.174661 100.584) (width 0.1524) (layer F.Cu) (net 27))
 (segment (start 151.174661 100.584) (end 151.13 100.584) (width 0.1524) (layer F.Cu) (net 27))
 (segment (start 151.948756 100.650989) (end 151.958989 100.650989) (width 0.1524) (layer F.Cu) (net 28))
 (segment (start 151.577526 100.279759) (end 151.948756 100.650989) (width 0.1524) (layer F.Cu) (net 28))
 (segment (start 154.559 106.68) (end 157.48 106.68) (width 0.1524) (layer F.Cu) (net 28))
 (segment (start 153.035 105.156) (end 154.559 106.68) (width 0.1524) (layer F.Cu) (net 28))
 (segment (start 151.577526 100.279759) (end 153.035 101.737233) (width 0.1524) (layer F.Cu) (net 28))
 (segment (start 153.035 101.737233) (end 153.035 105.156) (width 0.1524) (layer F.Cu) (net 28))
 (segment (start 154.559 104.14) (end 157.48 104.14) (width 0.1524) (layer F.Cu) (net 29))
 (segment (start 153.416 102.997) (end 154.559 104.14) (width 0.1524) (layer F.Cu) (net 29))
 (segment (start 151.931079 99.926207) (end 153.416 101.411128) (width 0.1524) (layer F.Cu) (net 29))
 (segment (start 153.416 101.411128) (end 153.416 102.997) (width 0.1524) (layer F.Cu) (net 29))
 (segment (start 152.655864 99.943882) (end 152.655864 99.950864) (width 0.1524) (layer F.Cu) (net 30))
 (segment (start 152.284634 99.572652) (end 152.655864 99.943882) (width 0.1524) (layer F.Cu) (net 30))
 (segment (start 154.305 101.6) (end 157.48 101.6) (width 0.1524) (layer F.Cu) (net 30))
 (segment (start 152.655864 99.950864) (end 154.305 101.6) (width 0.1524) (layer F.Cu) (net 30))
 (segment (start 155.956 97.536) (end 157.48 99.06) (width 0.1524) (layer F.Cu) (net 31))
 (segment (start 153.289 97.536) (end 155.956 97.536) (width 0.1524) (layer F.Cu) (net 31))
 (segment (start 152.285034 98.547749) (end 153.289 97.543783) (width 0.1524) (layer F.Cu) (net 31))
 (segment (start 153.289 97.543783) (end 153.289 97.536) (width 0.1524) (layer F.Cu) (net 31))
 (segment (start 153.543 96.52) (end 157.48 96.52) (width 0.1524) (layer F.Cu) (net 32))
 (segment (start 151.892 98.171) (end 153.543 96.52) (width 0.1524) (layer F.Cu) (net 32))
 (segment (start 151.931391 98.194106) (end 151.892 98.233497) (width 0.1524) (layer F.Cu) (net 32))
 (segment (start 151.892 98.233497) (end 151.892 98.171) (width 0.1524) (layer F.Cu) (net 32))
 (segment (start 153.924 93.98) (end 157.48 93.98) (width 0.1524) (layer F.Cu) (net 33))
 (segment (start 153.162 94.742) (end 153.924 93.98) (width 0.1524) (layer F.Cu) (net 33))
 (segment (start 153.162 96.266) (end 153.162 94.742) (width 0.1524) (layer F.Cu) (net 33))
 (segment (start 151.577749 97.840464) (end 151.577749 97.850251) (width 0.1524) (layer F.Cu) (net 33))
 (segment (start 151.577749 97.850251) (end 153.162 96.266) (width 0.1524) (layer F.Cu) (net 33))
 (segment (start 154.178 91.44) (end 157.48 91.44) (width 0.1524) (layer F.Cu) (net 34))
 (segment (start 152.4 93.218) (end 154.178 91.44) (width 0.1524) (layer F.Cu) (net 34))
 (segment (start 152.4 96.266) (end 152.4 93.218) (width 0.1524) (layer F.Cu) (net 34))
 (segment (start 151.224106 97.486821) (end 151.179179 97.486821) (width 0.1524) (layer F.Cu) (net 34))
 (segment (start 151.179179 97.486821) (end 152.4 96.266) (width 0.1524) (layer F.Cu) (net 34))
 (segment (start 154.178 88.9) (end 157.48 88.9) (width 0.1524) (layer F.Cu) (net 35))
 (segment (start 152.019 91.059) (end 154.178 88.9) (width 0.1524) (layer F.Cu) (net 35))
 (segment (start 152.019 95.885) (end 152.019 91.059) (width 0.1524) (layer F.Cu) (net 35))
 (segment (start 150.870464 97.133179) (end 150.770821 97.133179) (width 0.1524) (layer F.Cu) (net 35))
 (segment (start 150.770821 97.133179) (end 152.019 95.885) (width 0.1524) (layer F.Cu) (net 35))
 (segment (start 153.924 86.36) (end 157.48 86.36) (width 0.1524) (layer F.Cu) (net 36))
 (segment (start 151.638 88.646) (end 153.924 86.36) (width 0.1524) (layer F.Cu) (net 36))
 (segment (start 151.638 95.631) (end 151.638 88.646) (width 0.1524) (layer F.Cu) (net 36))
 (segment (start 150.495 96.774) (end 151.638 95.631) (width 0.1524) (layer F.Cu) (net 36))
 (segment (start 150.516821 96.779536) (end 150.500536 96.779536) (width 0.1524) (layer F.Cu) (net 36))
 (segment (start 150.500536 96.779536) (end 150.495 96.774) (width 0.1524) (layer F.Cu) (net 36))
 (segment (start 153.543 83.82) (end 157.48 83.82) (width 0.1524) (layer F.Cu) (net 37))
 (segment (start 151.257 86.106) (end 153.543 83.82) (width 0.1524) (layer F.Cu) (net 37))
 (segment (start 150.163179 96.425894) (end 151.257 95.332073) (width 0.1524) (layer F.Cu) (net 37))
 (segment (start 151.257 95.332073) (end 151.257 86.106) (width 0.1524) (layer F.Cu) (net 37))
 (segment (start 154.051 81.28) (end 157.48 81.28) (width 0.1524) (layer F.Cu) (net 38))
 (segment (start 150.876 84.455) (end 154.051 81.28) (width 0.1524) (layer F.Cu) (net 38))
 (segment (start 149.809536 96.072251) (end 150.876 95.005787) (width 0.1524) (layer F.Cu) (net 38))
 (segment (start 150.876 95.005787) (end 150.876 84.455) (width 0.1524) (layer F.Cu) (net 38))
 (segment (start 154.559 78.74) (end 157.48 78.74) (width 0.1524) (layer F.Cu) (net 39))
 (segment (start 150.495 82.804) (end 154.559 78.74) (width 0.1524) (layer F.Cu) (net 39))
 (segment (start 150.495 94.615) (end 150.495 82.804) (width 0.1524) (layer F.Cu) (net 39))
 (segment (start 149.606 95.504) (end 150.495 94.615) (width 0.1524) (layer F.Cu) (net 39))
 (segment (start 149.455894 95.718609) (end 149.606 95.568503) (width 0.1524) (layer F.Cu) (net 39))
 (segment (start 149.606 95.568503) (end 149.606 95.504) (width 0.1524) (layer F.Cu) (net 39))
 (segment (start 154.432 76.2) (end 157.48 76.2) (width 0.1524) (layer F.Cu) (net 40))
 (segment (start 150.114 80.518) (end 154.432 76.2) (width 0.1524) (layer F.Cu) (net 40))
 (segment (start 150.114 94.361) (end 150.114 80.518) (width 0.1524) (layer F.Cu) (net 40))
 (segment (start 149.102251 95.364966) (end 149.102251 95.372749) (width 0.1524) (layer F.Cu) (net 40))
 (segment (start 149.102251 95.372749) (end 150.114 94.361) (width 0.1524) (layer F.Cu) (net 40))
 (via (at 148.59 96.393) (size 0.6858) (drill 0.3302) (layers F.Cu B.Cu) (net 41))
 (segment (start 149.58702 97.39002) (end 148.59 96.393) (width 0.1524) (layer F.Cu) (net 41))
 (segment (start 148.59 99.06) (end 149.58702 98.06298) (width 0.1524) (layer F.Cu) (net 41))
 (segment (start 149.58702 98.06298) (end 149.58702 97.39002) (width 0.1524) (layer F.Cu) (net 41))
 (segment (start 148.59 95.908067) (end 148.463 95.781067) (width 0.1524) (layer B.Cu) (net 41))
 (segment (start 148.59 96.393) (end 148.59 95.908067) (width 0.1524) (layer B.Cu) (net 41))
 (via (at 148.463 92.837) (size 0.6858) (drill 0.3302) (layers F.Cu B.Cu) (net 41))
 (segment (start 148.463 95.781067) (end 148.463 92.837) (width 0.1524) (layer B.Cu) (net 41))
 (segment (start 148.463 92.837) (end 148.463 77.216) (width 0.1524) (layer F.Cu) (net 41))
 (segment (start 152.019 73.66) (end 157.48 73.66) (width 0.1524) (layer F.Cu) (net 41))
 (segment (start 148.463 77.216) (end 152.019 73.66) (width 0.1524) (layer F.Cu) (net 41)))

